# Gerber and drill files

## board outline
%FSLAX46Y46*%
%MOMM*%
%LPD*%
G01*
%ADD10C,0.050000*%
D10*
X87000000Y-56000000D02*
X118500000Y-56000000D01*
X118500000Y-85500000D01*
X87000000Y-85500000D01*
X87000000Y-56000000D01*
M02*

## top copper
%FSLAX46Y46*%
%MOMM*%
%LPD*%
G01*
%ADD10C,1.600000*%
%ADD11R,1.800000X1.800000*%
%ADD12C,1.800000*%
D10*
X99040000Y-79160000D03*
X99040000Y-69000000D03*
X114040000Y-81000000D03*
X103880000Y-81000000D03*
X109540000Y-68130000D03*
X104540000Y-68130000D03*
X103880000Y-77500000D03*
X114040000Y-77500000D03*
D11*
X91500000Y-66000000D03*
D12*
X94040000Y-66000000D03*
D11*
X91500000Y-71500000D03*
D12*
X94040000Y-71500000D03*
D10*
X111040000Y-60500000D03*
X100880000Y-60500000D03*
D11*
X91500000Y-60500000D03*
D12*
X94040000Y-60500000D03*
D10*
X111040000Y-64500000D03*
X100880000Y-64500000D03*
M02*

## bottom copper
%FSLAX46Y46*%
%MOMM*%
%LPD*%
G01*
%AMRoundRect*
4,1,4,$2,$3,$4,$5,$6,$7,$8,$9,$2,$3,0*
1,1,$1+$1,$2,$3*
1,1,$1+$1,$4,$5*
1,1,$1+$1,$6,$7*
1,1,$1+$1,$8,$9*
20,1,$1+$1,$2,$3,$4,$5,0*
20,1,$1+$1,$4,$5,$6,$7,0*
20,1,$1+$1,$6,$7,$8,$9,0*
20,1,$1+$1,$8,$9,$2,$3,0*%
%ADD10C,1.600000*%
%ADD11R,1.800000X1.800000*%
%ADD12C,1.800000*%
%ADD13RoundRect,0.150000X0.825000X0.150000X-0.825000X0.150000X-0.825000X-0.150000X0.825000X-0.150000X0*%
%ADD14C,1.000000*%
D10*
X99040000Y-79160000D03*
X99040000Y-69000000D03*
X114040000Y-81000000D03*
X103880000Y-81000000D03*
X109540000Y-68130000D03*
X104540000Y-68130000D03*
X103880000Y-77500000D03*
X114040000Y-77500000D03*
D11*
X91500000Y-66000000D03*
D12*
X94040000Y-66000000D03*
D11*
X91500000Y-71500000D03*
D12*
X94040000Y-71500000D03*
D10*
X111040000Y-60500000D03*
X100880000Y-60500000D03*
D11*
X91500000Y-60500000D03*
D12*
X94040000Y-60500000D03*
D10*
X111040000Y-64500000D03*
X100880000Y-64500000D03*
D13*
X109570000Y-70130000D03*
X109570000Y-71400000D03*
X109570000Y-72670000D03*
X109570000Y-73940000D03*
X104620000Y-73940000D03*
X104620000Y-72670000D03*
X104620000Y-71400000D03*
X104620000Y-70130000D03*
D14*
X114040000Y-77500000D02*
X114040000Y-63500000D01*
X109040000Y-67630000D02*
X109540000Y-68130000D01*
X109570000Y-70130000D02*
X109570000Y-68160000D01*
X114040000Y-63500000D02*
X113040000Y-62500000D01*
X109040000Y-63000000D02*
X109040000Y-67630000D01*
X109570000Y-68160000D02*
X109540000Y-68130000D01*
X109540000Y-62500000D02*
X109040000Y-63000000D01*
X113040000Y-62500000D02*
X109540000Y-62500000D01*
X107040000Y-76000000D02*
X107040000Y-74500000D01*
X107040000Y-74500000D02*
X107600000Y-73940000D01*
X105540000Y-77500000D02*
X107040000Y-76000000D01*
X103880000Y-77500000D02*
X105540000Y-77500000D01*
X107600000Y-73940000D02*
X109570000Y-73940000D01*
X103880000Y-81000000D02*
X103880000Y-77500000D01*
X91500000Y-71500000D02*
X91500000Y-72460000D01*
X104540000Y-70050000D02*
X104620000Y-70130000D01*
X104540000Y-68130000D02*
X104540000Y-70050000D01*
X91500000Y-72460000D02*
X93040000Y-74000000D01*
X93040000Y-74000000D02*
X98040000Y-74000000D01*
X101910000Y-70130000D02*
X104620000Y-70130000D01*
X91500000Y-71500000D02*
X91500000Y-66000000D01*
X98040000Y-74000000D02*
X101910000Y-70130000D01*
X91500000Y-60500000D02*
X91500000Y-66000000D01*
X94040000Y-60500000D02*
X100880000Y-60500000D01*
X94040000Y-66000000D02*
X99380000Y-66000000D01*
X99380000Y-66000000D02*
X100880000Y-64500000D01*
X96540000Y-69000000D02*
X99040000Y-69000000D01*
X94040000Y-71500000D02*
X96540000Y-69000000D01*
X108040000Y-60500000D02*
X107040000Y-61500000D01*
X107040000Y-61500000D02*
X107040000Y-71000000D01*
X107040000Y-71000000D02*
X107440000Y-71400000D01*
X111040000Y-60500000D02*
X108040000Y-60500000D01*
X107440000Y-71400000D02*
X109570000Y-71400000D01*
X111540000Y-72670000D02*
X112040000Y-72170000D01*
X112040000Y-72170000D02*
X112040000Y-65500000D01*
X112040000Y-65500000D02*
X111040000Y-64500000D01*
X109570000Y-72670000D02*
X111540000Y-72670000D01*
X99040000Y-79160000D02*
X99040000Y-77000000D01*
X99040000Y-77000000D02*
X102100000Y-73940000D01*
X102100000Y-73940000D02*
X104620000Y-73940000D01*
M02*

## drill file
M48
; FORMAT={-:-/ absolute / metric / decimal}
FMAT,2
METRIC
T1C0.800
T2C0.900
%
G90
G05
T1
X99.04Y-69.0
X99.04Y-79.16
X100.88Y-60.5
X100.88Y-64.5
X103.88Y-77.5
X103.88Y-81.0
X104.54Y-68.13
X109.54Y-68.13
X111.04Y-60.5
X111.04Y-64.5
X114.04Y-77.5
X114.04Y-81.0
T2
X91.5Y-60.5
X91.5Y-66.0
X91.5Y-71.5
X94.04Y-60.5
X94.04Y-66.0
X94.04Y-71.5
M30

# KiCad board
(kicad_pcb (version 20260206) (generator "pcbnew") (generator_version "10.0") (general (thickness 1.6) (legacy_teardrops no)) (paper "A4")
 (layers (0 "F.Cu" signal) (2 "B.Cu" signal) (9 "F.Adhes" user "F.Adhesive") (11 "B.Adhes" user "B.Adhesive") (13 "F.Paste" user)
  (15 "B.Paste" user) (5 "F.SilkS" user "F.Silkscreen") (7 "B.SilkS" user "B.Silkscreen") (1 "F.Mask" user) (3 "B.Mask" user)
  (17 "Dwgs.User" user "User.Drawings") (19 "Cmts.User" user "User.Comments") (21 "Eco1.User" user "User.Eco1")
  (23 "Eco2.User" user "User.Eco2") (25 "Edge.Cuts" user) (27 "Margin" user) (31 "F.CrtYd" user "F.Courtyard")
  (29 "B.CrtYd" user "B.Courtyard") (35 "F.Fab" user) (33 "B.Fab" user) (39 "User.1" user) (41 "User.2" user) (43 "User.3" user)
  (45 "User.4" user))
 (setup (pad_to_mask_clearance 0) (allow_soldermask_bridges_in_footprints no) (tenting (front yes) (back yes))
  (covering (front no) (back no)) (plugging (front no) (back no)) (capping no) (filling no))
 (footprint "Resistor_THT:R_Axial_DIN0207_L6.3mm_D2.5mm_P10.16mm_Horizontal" (layer "F.Cu") (at 99.04 79.16 90)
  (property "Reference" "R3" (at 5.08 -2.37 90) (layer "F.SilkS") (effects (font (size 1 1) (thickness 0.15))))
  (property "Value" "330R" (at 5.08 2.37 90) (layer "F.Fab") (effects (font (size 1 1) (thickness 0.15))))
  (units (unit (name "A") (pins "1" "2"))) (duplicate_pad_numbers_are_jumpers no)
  (pad "1" thru_hole circle (at 0 0 90) (size 1.6 1.6) (drill 0.8) (layers "*.Cu" "*.Mask") (remove_unused_layers no) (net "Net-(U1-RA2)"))
  (pad "2" thru_hole circle (at 10.16 0 90) (size 1.6 1.6) (drill 0.8) (layers "*.Cu" "*.Mask") (remove_unused_layers no) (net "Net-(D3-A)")))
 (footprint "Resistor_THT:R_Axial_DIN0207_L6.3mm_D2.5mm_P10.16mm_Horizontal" (layer "F.Cu") (at 114.04 81 180)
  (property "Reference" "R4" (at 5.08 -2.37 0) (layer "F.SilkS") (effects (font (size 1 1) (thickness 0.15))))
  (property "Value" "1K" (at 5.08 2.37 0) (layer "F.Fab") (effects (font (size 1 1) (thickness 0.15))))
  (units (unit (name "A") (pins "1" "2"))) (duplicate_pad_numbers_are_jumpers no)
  (pad "1" thru_hole circle (at 0 0 180) (size 1.6 1.6) (drill 0.8) (layers "*.Cu" "*.Mask") (remove_unused_layers no)
   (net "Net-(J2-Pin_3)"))
  (pad "2" thru_hole circle (at 10.16 0 180) (size 1.6 1.6) (drill 0.8) (layers "*.Cu" "*.Mask") (remove_unused_layers no)
   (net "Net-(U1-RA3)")))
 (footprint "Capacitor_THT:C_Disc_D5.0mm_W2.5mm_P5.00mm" (layer "F.Cu") (at 109.54 68.13 180)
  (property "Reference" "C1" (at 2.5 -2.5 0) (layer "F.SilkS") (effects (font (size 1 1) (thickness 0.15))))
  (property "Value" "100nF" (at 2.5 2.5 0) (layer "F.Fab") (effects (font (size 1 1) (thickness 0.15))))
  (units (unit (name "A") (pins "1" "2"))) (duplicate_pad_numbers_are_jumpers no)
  (pad "1" thru_hole circle (at 0 0 180) (size 1.6 1.6) (drill 0.8) (layers "*.Cu" "*.Mask") (remove_unused_layers no) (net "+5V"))
  (pad "2" thru_hole circle (at 5 0 180) (size 1.6 1.6) (drill 0.8) (layers "*.Cu" "*.Mask") (remove_unused_layers no) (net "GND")))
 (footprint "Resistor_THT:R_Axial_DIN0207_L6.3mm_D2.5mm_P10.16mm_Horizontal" (layer "F.Cu") (at 103.88 77.5)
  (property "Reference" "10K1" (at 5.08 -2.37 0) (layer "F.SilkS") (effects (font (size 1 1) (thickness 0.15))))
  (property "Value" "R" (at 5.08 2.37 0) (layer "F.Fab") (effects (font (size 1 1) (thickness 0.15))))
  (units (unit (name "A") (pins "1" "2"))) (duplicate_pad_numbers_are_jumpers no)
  (pad "1" thru_hole circle (at 0 0) (size 1.6 1.6) (drill 0.8) (layers "*.Cu" "*.Mask") (remove_unused_layers no) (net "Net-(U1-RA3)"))
  (pad "2" thru_hole circle (at 10.16 0) (size 1.6 1.6) (drill 0.8) (layers "*.Cu" "*.Mask") (remove_unused_layers no) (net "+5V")))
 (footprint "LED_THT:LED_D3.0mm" (layer "F.Cu") (at 91.5 66)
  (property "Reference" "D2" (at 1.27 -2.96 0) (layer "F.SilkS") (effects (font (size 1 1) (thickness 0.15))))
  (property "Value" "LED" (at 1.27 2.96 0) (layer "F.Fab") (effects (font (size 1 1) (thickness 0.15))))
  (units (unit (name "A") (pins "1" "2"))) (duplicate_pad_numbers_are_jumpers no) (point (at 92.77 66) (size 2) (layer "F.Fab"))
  (pad "1" thru_hole rect (at 0 0) (size 1.8 1.8) (drill 0.9) (layers "*.Cu" "*.Mask") (remove_unused_layers no) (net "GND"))
  (pad "2" thru_hole circle (at 2.54 0) (size 1.8 1.8) (drill 0.9) (layers "*.Cu" "*.Mask") (remove_unused_layers no) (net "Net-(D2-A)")))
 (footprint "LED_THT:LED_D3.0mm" (layer "F.Cu") (at 91.5 71.5)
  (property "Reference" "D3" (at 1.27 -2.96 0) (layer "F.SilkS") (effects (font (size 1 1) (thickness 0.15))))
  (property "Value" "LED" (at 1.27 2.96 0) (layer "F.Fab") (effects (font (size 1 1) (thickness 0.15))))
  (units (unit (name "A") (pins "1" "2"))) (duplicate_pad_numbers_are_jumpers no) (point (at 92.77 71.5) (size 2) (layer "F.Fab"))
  (pad "1" thru_hole rect (at 0 0) (size 1.8 1.8) (drill 0.9) (layers "*.Cu" "*.Mask") (remove_unused_layers no) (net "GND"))
  (pad "2" thru_hole circle (at 2.54 0) (size 1.8 1.8) (drill 0.9) (layers "*.Cu" "*.Mask") (remove_unused_layers no) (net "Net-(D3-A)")))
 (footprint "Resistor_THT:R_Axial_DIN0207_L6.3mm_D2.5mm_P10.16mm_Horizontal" (layer "F.Cu") (at 111.04 60.5 180)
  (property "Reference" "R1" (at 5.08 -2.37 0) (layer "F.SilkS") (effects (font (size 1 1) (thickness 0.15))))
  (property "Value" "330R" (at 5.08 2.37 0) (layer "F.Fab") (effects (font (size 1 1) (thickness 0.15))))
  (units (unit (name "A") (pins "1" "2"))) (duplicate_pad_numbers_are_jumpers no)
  (pad "1" thru_hole circle (at 0 0 180) (size 1.6 1.6) (drill 0.8) (layers "*.Cu" "*.Mask") (remove_unused_layers no) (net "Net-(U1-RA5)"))
  (pad "2" thru_hole circle (at 10.16 0 180) (size 1.6 1.6) (drill 0.8) (layers "*.Cu" "*.Mask") (remove_unused_layers no)
   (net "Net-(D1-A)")))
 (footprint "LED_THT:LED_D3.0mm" (layer "F.Cu") (at 91.5 60.5)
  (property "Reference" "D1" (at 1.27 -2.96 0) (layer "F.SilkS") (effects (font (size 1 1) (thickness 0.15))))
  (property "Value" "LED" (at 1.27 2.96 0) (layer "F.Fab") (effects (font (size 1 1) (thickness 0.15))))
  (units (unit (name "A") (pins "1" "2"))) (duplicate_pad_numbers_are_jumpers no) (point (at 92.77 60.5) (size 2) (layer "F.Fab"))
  (pad "1" thru_hole rect (at 0 0) (size 1.8 1.8) (drill 0.9) (layers "*.Cu" "*.Mask") (remove_unused_layers no) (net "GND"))
  (pad "2" thru_hole circle (at 2.54 0) (size 1.8 1.8) (drill 0.9) (layers "*.Cu" "*.Mask") (remove_unused_layers no) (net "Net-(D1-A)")))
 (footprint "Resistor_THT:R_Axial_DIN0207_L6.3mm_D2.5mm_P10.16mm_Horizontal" (layer "F.Cu") (at 111.04 64.5 180)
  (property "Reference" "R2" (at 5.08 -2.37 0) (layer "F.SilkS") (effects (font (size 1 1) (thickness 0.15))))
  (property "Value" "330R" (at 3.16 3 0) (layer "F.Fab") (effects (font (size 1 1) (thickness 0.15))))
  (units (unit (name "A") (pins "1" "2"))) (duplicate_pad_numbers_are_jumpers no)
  (pad "1" thru_hole circle (at 0 0 180) (size 1.6 1.6) (drill 0.8) (layers "*.Cu" "*.Mask") (remove_unused_layers no) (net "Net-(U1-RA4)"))
  (pad "2" thru_hole circle (at 10.16 0 180) (size 1.6 1.6) (drill 0.8) (layers "*.Cu" "*.Mask") (remove_unused_layers no)
   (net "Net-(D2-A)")))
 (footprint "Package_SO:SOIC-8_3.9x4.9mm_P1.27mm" (layer "B.Cu") (at 107.095 72.035 180)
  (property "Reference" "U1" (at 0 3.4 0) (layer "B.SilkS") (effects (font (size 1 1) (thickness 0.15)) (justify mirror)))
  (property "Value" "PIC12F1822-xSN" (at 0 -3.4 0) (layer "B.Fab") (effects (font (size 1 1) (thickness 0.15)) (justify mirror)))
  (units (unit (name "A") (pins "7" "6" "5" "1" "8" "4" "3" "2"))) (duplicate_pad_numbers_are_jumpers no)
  (pad "1" smd roundrect (at -2.475 1.905 180) (size 1.95 0.6) (layers "B.Cu" "B.Mask" "B.Paste") (roundrect_rratio 0.25) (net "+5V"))
  (pad "2" smd roundrect (at -2.475 0.635 180) (size 1.95 0.6) (layers "B.Cu" "B.Mask" "B.Paste") (roundrect_rratio 0.25)
   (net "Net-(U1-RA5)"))
  (pad "3" smd roundrect (at -2.475 -0.635 180) (size 1.95 0.6) (layers "B.Cu" "B.Mask" "B.Paste") (roundrect_rratio 0.25)
   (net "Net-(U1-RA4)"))
  (pad "4" smd roundrect (at -2.475 -1.905 180) (size 1.95 0.6) (layers "B.Cu" "B.Mask" "B.Paste") (roundrect_rratio 0.25)
   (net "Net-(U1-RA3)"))
  (pad "5" smd roundrect (at 2.475 -1.905 180) (size 1.95 0.6) (layers "B.Cu" "B.Mask" "B.Paste") (roundrect_rratio 0.25)
   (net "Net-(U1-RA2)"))
  (pad "6" smd roundrect (at 2.475 -0.635 180) (size 1.95 0.6) (layers "B.Cu" "B.Mask" "B.Paste") (roundrect_rratio 0.25)
   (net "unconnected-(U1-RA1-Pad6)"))
  (pad "7" smd roundrect (at 2.475 0.635 180) (size 1.95 0.6) (layers "B.Cu" "B.Mask" "B.Paste") (roundrect_rratio 0.25)
   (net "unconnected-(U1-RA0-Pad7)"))
  (pad "8" smd roundrect (at 2.475 1.905 180) (size 1.95 0.6) (layers "B.Cu" "B.Mask" "B.Paste") (roundrect_rratio 0.25) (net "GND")))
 (gr_rect (start 87 56) (end 118.5 85.5) (stroke (width 0.05) (type default)) (fill no) (layer "Edge.Cuts"))
 (segment (start 114.04 77.5) (end 114.04 63.5) (width 1) (layer "B.Cu") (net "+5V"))
 (segment (start 109.04 67.63) (end 109.54 68.13) (width 1) (layer "B.Cu") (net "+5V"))
 (segment (start 109.57 70.13) (end 109.57 68.16) (width 1) (layer "B.Cu") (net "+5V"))
 (segment (start 114.04 63.5) (end 113.04 62.5) (width 1) (layer "B.Cu") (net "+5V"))
 (segment (start 109.04 63) (end 109.04 67.63) (width 1) (layer "B.Cu") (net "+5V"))
 (segment (start 109.57 68.16) (end 109.54 68.13) (width 1) (layer "B.Cu") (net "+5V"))
 (segment (start 109.54 62.5) (end 109.04 63) (width 1) (layer "B.Cu") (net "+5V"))
 (segment (start 113.04 62.5) (end 109.54 62.5) (width 1) (layer "B.Cu") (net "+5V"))
 (segment (start 107.04 76) (end 107.04 74.5) (width 1) (layer "B.Cu") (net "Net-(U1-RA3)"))
 (segment (start 107.04 74.5) (end 107.6 73.94) (width 1) (layer "B.Cu") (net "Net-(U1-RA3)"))
 (segment (start 105.54 77.5) (end 107.04 76) (width 1) (layer "B.Cu") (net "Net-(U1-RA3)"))
 (segment (start 103.88 77.5) (end 105.54 77.5) (width 1) (layer "B.Cu") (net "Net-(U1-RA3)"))
 (segment (start 107.6 73.94) (end 109.57 73.94) (width 1) (layer "B.Cu") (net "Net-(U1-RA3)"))
 (segment (start 103.88 81) (end 103.88 77.5) (width 1) (layer "B.Cu") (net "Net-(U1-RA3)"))
 (segment (start 91.5 71.5) (end 91.5 72.46) (width 1) (layer "B.Cu") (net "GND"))
 (segment (start 104.54 70.05) (end 104.62 70.13) (width 1) (layer "B.Cu") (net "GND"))
 (segment (start 104.54 68.13) (end 104.54 70.05) (width 1) (layer "B.Cu") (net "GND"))
 (segment (start 91.5 72.46) (end 93.04 74) (width 1) (layer "B.Cu") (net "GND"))
 (segment (start 93.04 74) (end 98.04 74) (width 1) (layer "B.Cu") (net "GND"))
 (segment (start 101.91 70.13) (end 104.62 70.13) (width 1) (layer "B.Cu") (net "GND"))
 (segment (start 91.5 71.5) (end 91.5 66) (width 1) (layer "B.Cu") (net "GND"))
 (segment (start 98.04 74) (end 101.91 70.13) (width 1) (layer "B.Cu") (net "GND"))
 (segment (start 91.5 60.5) (end 91.5 66) (width 1) (layer "B.Cu") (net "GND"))
 (segment (start 94.04 60.5) (end 100.88 60.5) (width 1) (layer "B.Cu") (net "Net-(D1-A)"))
 (segment (start 94.04 66) (end 99.38 66) (width 1) (layer "B.Cu") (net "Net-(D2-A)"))
 (segment (start 99.38 66) (end 100.88 64.5) (width 1) (layer "B.Cu") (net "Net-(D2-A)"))
 (segment (start 96.54 69) (end 99.04 69) (width 1) (layer "B.Cu") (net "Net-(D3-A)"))
 (segment (start 94.04 71.5) (end 96.54 69) (width 1) (layer "B.Cu") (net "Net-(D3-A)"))
 (segment (start 108.04 60.5) (end 107.04 61.5) (width 1) (layer "B.Cu") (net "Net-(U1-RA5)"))
 (segment (start 107.04 61.5) (end 107.04 71) (width 1) (layer "B.Cu") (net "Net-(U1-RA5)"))
 (segment (start 107.04 71) (end 107.44 71.4) (width 1) (layer "B.Cu") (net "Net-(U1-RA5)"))
 (segment (start 111.04 60.5) (end 108.04 60.5) (width 1) (layer "B.Cu") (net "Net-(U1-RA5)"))
 (segment (start 107.44 71.4) (end 109.57 71.4) (width 1) (layer "B.Cu") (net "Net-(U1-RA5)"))
 (segment (start 111.54 72.67) (end 112.04 72.17) (width 1) (layer "B.Cu") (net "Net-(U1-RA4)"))
 (segment (start 112.04 72.17) (end 112.04 65.5) (width 1) (layer "B.Cu") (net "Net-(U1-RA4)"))
 (segment (start 112.04 65.5) (end 111.04 64.5) (width 1) (layer "B.Cu") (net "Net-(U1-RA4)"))
 (segment (start 109.57 72.67) (end 111.54 72.67) (width 1) (layer "B.Cu") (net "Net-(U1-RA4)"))
 (segment (start 99.04 79.16) (end 99.04 77) (width 1) (layer "B.Cu") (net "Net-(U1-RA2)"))
 (segment (start 99.04 77) (end 102.1 73.94) (width 1) (layer "B.Cu") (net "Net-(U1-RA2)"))
 (segment (start 102.1 73.94) (end 104.62 73.94) (width 1) (layer "B.Cu") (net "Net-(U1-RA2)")))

